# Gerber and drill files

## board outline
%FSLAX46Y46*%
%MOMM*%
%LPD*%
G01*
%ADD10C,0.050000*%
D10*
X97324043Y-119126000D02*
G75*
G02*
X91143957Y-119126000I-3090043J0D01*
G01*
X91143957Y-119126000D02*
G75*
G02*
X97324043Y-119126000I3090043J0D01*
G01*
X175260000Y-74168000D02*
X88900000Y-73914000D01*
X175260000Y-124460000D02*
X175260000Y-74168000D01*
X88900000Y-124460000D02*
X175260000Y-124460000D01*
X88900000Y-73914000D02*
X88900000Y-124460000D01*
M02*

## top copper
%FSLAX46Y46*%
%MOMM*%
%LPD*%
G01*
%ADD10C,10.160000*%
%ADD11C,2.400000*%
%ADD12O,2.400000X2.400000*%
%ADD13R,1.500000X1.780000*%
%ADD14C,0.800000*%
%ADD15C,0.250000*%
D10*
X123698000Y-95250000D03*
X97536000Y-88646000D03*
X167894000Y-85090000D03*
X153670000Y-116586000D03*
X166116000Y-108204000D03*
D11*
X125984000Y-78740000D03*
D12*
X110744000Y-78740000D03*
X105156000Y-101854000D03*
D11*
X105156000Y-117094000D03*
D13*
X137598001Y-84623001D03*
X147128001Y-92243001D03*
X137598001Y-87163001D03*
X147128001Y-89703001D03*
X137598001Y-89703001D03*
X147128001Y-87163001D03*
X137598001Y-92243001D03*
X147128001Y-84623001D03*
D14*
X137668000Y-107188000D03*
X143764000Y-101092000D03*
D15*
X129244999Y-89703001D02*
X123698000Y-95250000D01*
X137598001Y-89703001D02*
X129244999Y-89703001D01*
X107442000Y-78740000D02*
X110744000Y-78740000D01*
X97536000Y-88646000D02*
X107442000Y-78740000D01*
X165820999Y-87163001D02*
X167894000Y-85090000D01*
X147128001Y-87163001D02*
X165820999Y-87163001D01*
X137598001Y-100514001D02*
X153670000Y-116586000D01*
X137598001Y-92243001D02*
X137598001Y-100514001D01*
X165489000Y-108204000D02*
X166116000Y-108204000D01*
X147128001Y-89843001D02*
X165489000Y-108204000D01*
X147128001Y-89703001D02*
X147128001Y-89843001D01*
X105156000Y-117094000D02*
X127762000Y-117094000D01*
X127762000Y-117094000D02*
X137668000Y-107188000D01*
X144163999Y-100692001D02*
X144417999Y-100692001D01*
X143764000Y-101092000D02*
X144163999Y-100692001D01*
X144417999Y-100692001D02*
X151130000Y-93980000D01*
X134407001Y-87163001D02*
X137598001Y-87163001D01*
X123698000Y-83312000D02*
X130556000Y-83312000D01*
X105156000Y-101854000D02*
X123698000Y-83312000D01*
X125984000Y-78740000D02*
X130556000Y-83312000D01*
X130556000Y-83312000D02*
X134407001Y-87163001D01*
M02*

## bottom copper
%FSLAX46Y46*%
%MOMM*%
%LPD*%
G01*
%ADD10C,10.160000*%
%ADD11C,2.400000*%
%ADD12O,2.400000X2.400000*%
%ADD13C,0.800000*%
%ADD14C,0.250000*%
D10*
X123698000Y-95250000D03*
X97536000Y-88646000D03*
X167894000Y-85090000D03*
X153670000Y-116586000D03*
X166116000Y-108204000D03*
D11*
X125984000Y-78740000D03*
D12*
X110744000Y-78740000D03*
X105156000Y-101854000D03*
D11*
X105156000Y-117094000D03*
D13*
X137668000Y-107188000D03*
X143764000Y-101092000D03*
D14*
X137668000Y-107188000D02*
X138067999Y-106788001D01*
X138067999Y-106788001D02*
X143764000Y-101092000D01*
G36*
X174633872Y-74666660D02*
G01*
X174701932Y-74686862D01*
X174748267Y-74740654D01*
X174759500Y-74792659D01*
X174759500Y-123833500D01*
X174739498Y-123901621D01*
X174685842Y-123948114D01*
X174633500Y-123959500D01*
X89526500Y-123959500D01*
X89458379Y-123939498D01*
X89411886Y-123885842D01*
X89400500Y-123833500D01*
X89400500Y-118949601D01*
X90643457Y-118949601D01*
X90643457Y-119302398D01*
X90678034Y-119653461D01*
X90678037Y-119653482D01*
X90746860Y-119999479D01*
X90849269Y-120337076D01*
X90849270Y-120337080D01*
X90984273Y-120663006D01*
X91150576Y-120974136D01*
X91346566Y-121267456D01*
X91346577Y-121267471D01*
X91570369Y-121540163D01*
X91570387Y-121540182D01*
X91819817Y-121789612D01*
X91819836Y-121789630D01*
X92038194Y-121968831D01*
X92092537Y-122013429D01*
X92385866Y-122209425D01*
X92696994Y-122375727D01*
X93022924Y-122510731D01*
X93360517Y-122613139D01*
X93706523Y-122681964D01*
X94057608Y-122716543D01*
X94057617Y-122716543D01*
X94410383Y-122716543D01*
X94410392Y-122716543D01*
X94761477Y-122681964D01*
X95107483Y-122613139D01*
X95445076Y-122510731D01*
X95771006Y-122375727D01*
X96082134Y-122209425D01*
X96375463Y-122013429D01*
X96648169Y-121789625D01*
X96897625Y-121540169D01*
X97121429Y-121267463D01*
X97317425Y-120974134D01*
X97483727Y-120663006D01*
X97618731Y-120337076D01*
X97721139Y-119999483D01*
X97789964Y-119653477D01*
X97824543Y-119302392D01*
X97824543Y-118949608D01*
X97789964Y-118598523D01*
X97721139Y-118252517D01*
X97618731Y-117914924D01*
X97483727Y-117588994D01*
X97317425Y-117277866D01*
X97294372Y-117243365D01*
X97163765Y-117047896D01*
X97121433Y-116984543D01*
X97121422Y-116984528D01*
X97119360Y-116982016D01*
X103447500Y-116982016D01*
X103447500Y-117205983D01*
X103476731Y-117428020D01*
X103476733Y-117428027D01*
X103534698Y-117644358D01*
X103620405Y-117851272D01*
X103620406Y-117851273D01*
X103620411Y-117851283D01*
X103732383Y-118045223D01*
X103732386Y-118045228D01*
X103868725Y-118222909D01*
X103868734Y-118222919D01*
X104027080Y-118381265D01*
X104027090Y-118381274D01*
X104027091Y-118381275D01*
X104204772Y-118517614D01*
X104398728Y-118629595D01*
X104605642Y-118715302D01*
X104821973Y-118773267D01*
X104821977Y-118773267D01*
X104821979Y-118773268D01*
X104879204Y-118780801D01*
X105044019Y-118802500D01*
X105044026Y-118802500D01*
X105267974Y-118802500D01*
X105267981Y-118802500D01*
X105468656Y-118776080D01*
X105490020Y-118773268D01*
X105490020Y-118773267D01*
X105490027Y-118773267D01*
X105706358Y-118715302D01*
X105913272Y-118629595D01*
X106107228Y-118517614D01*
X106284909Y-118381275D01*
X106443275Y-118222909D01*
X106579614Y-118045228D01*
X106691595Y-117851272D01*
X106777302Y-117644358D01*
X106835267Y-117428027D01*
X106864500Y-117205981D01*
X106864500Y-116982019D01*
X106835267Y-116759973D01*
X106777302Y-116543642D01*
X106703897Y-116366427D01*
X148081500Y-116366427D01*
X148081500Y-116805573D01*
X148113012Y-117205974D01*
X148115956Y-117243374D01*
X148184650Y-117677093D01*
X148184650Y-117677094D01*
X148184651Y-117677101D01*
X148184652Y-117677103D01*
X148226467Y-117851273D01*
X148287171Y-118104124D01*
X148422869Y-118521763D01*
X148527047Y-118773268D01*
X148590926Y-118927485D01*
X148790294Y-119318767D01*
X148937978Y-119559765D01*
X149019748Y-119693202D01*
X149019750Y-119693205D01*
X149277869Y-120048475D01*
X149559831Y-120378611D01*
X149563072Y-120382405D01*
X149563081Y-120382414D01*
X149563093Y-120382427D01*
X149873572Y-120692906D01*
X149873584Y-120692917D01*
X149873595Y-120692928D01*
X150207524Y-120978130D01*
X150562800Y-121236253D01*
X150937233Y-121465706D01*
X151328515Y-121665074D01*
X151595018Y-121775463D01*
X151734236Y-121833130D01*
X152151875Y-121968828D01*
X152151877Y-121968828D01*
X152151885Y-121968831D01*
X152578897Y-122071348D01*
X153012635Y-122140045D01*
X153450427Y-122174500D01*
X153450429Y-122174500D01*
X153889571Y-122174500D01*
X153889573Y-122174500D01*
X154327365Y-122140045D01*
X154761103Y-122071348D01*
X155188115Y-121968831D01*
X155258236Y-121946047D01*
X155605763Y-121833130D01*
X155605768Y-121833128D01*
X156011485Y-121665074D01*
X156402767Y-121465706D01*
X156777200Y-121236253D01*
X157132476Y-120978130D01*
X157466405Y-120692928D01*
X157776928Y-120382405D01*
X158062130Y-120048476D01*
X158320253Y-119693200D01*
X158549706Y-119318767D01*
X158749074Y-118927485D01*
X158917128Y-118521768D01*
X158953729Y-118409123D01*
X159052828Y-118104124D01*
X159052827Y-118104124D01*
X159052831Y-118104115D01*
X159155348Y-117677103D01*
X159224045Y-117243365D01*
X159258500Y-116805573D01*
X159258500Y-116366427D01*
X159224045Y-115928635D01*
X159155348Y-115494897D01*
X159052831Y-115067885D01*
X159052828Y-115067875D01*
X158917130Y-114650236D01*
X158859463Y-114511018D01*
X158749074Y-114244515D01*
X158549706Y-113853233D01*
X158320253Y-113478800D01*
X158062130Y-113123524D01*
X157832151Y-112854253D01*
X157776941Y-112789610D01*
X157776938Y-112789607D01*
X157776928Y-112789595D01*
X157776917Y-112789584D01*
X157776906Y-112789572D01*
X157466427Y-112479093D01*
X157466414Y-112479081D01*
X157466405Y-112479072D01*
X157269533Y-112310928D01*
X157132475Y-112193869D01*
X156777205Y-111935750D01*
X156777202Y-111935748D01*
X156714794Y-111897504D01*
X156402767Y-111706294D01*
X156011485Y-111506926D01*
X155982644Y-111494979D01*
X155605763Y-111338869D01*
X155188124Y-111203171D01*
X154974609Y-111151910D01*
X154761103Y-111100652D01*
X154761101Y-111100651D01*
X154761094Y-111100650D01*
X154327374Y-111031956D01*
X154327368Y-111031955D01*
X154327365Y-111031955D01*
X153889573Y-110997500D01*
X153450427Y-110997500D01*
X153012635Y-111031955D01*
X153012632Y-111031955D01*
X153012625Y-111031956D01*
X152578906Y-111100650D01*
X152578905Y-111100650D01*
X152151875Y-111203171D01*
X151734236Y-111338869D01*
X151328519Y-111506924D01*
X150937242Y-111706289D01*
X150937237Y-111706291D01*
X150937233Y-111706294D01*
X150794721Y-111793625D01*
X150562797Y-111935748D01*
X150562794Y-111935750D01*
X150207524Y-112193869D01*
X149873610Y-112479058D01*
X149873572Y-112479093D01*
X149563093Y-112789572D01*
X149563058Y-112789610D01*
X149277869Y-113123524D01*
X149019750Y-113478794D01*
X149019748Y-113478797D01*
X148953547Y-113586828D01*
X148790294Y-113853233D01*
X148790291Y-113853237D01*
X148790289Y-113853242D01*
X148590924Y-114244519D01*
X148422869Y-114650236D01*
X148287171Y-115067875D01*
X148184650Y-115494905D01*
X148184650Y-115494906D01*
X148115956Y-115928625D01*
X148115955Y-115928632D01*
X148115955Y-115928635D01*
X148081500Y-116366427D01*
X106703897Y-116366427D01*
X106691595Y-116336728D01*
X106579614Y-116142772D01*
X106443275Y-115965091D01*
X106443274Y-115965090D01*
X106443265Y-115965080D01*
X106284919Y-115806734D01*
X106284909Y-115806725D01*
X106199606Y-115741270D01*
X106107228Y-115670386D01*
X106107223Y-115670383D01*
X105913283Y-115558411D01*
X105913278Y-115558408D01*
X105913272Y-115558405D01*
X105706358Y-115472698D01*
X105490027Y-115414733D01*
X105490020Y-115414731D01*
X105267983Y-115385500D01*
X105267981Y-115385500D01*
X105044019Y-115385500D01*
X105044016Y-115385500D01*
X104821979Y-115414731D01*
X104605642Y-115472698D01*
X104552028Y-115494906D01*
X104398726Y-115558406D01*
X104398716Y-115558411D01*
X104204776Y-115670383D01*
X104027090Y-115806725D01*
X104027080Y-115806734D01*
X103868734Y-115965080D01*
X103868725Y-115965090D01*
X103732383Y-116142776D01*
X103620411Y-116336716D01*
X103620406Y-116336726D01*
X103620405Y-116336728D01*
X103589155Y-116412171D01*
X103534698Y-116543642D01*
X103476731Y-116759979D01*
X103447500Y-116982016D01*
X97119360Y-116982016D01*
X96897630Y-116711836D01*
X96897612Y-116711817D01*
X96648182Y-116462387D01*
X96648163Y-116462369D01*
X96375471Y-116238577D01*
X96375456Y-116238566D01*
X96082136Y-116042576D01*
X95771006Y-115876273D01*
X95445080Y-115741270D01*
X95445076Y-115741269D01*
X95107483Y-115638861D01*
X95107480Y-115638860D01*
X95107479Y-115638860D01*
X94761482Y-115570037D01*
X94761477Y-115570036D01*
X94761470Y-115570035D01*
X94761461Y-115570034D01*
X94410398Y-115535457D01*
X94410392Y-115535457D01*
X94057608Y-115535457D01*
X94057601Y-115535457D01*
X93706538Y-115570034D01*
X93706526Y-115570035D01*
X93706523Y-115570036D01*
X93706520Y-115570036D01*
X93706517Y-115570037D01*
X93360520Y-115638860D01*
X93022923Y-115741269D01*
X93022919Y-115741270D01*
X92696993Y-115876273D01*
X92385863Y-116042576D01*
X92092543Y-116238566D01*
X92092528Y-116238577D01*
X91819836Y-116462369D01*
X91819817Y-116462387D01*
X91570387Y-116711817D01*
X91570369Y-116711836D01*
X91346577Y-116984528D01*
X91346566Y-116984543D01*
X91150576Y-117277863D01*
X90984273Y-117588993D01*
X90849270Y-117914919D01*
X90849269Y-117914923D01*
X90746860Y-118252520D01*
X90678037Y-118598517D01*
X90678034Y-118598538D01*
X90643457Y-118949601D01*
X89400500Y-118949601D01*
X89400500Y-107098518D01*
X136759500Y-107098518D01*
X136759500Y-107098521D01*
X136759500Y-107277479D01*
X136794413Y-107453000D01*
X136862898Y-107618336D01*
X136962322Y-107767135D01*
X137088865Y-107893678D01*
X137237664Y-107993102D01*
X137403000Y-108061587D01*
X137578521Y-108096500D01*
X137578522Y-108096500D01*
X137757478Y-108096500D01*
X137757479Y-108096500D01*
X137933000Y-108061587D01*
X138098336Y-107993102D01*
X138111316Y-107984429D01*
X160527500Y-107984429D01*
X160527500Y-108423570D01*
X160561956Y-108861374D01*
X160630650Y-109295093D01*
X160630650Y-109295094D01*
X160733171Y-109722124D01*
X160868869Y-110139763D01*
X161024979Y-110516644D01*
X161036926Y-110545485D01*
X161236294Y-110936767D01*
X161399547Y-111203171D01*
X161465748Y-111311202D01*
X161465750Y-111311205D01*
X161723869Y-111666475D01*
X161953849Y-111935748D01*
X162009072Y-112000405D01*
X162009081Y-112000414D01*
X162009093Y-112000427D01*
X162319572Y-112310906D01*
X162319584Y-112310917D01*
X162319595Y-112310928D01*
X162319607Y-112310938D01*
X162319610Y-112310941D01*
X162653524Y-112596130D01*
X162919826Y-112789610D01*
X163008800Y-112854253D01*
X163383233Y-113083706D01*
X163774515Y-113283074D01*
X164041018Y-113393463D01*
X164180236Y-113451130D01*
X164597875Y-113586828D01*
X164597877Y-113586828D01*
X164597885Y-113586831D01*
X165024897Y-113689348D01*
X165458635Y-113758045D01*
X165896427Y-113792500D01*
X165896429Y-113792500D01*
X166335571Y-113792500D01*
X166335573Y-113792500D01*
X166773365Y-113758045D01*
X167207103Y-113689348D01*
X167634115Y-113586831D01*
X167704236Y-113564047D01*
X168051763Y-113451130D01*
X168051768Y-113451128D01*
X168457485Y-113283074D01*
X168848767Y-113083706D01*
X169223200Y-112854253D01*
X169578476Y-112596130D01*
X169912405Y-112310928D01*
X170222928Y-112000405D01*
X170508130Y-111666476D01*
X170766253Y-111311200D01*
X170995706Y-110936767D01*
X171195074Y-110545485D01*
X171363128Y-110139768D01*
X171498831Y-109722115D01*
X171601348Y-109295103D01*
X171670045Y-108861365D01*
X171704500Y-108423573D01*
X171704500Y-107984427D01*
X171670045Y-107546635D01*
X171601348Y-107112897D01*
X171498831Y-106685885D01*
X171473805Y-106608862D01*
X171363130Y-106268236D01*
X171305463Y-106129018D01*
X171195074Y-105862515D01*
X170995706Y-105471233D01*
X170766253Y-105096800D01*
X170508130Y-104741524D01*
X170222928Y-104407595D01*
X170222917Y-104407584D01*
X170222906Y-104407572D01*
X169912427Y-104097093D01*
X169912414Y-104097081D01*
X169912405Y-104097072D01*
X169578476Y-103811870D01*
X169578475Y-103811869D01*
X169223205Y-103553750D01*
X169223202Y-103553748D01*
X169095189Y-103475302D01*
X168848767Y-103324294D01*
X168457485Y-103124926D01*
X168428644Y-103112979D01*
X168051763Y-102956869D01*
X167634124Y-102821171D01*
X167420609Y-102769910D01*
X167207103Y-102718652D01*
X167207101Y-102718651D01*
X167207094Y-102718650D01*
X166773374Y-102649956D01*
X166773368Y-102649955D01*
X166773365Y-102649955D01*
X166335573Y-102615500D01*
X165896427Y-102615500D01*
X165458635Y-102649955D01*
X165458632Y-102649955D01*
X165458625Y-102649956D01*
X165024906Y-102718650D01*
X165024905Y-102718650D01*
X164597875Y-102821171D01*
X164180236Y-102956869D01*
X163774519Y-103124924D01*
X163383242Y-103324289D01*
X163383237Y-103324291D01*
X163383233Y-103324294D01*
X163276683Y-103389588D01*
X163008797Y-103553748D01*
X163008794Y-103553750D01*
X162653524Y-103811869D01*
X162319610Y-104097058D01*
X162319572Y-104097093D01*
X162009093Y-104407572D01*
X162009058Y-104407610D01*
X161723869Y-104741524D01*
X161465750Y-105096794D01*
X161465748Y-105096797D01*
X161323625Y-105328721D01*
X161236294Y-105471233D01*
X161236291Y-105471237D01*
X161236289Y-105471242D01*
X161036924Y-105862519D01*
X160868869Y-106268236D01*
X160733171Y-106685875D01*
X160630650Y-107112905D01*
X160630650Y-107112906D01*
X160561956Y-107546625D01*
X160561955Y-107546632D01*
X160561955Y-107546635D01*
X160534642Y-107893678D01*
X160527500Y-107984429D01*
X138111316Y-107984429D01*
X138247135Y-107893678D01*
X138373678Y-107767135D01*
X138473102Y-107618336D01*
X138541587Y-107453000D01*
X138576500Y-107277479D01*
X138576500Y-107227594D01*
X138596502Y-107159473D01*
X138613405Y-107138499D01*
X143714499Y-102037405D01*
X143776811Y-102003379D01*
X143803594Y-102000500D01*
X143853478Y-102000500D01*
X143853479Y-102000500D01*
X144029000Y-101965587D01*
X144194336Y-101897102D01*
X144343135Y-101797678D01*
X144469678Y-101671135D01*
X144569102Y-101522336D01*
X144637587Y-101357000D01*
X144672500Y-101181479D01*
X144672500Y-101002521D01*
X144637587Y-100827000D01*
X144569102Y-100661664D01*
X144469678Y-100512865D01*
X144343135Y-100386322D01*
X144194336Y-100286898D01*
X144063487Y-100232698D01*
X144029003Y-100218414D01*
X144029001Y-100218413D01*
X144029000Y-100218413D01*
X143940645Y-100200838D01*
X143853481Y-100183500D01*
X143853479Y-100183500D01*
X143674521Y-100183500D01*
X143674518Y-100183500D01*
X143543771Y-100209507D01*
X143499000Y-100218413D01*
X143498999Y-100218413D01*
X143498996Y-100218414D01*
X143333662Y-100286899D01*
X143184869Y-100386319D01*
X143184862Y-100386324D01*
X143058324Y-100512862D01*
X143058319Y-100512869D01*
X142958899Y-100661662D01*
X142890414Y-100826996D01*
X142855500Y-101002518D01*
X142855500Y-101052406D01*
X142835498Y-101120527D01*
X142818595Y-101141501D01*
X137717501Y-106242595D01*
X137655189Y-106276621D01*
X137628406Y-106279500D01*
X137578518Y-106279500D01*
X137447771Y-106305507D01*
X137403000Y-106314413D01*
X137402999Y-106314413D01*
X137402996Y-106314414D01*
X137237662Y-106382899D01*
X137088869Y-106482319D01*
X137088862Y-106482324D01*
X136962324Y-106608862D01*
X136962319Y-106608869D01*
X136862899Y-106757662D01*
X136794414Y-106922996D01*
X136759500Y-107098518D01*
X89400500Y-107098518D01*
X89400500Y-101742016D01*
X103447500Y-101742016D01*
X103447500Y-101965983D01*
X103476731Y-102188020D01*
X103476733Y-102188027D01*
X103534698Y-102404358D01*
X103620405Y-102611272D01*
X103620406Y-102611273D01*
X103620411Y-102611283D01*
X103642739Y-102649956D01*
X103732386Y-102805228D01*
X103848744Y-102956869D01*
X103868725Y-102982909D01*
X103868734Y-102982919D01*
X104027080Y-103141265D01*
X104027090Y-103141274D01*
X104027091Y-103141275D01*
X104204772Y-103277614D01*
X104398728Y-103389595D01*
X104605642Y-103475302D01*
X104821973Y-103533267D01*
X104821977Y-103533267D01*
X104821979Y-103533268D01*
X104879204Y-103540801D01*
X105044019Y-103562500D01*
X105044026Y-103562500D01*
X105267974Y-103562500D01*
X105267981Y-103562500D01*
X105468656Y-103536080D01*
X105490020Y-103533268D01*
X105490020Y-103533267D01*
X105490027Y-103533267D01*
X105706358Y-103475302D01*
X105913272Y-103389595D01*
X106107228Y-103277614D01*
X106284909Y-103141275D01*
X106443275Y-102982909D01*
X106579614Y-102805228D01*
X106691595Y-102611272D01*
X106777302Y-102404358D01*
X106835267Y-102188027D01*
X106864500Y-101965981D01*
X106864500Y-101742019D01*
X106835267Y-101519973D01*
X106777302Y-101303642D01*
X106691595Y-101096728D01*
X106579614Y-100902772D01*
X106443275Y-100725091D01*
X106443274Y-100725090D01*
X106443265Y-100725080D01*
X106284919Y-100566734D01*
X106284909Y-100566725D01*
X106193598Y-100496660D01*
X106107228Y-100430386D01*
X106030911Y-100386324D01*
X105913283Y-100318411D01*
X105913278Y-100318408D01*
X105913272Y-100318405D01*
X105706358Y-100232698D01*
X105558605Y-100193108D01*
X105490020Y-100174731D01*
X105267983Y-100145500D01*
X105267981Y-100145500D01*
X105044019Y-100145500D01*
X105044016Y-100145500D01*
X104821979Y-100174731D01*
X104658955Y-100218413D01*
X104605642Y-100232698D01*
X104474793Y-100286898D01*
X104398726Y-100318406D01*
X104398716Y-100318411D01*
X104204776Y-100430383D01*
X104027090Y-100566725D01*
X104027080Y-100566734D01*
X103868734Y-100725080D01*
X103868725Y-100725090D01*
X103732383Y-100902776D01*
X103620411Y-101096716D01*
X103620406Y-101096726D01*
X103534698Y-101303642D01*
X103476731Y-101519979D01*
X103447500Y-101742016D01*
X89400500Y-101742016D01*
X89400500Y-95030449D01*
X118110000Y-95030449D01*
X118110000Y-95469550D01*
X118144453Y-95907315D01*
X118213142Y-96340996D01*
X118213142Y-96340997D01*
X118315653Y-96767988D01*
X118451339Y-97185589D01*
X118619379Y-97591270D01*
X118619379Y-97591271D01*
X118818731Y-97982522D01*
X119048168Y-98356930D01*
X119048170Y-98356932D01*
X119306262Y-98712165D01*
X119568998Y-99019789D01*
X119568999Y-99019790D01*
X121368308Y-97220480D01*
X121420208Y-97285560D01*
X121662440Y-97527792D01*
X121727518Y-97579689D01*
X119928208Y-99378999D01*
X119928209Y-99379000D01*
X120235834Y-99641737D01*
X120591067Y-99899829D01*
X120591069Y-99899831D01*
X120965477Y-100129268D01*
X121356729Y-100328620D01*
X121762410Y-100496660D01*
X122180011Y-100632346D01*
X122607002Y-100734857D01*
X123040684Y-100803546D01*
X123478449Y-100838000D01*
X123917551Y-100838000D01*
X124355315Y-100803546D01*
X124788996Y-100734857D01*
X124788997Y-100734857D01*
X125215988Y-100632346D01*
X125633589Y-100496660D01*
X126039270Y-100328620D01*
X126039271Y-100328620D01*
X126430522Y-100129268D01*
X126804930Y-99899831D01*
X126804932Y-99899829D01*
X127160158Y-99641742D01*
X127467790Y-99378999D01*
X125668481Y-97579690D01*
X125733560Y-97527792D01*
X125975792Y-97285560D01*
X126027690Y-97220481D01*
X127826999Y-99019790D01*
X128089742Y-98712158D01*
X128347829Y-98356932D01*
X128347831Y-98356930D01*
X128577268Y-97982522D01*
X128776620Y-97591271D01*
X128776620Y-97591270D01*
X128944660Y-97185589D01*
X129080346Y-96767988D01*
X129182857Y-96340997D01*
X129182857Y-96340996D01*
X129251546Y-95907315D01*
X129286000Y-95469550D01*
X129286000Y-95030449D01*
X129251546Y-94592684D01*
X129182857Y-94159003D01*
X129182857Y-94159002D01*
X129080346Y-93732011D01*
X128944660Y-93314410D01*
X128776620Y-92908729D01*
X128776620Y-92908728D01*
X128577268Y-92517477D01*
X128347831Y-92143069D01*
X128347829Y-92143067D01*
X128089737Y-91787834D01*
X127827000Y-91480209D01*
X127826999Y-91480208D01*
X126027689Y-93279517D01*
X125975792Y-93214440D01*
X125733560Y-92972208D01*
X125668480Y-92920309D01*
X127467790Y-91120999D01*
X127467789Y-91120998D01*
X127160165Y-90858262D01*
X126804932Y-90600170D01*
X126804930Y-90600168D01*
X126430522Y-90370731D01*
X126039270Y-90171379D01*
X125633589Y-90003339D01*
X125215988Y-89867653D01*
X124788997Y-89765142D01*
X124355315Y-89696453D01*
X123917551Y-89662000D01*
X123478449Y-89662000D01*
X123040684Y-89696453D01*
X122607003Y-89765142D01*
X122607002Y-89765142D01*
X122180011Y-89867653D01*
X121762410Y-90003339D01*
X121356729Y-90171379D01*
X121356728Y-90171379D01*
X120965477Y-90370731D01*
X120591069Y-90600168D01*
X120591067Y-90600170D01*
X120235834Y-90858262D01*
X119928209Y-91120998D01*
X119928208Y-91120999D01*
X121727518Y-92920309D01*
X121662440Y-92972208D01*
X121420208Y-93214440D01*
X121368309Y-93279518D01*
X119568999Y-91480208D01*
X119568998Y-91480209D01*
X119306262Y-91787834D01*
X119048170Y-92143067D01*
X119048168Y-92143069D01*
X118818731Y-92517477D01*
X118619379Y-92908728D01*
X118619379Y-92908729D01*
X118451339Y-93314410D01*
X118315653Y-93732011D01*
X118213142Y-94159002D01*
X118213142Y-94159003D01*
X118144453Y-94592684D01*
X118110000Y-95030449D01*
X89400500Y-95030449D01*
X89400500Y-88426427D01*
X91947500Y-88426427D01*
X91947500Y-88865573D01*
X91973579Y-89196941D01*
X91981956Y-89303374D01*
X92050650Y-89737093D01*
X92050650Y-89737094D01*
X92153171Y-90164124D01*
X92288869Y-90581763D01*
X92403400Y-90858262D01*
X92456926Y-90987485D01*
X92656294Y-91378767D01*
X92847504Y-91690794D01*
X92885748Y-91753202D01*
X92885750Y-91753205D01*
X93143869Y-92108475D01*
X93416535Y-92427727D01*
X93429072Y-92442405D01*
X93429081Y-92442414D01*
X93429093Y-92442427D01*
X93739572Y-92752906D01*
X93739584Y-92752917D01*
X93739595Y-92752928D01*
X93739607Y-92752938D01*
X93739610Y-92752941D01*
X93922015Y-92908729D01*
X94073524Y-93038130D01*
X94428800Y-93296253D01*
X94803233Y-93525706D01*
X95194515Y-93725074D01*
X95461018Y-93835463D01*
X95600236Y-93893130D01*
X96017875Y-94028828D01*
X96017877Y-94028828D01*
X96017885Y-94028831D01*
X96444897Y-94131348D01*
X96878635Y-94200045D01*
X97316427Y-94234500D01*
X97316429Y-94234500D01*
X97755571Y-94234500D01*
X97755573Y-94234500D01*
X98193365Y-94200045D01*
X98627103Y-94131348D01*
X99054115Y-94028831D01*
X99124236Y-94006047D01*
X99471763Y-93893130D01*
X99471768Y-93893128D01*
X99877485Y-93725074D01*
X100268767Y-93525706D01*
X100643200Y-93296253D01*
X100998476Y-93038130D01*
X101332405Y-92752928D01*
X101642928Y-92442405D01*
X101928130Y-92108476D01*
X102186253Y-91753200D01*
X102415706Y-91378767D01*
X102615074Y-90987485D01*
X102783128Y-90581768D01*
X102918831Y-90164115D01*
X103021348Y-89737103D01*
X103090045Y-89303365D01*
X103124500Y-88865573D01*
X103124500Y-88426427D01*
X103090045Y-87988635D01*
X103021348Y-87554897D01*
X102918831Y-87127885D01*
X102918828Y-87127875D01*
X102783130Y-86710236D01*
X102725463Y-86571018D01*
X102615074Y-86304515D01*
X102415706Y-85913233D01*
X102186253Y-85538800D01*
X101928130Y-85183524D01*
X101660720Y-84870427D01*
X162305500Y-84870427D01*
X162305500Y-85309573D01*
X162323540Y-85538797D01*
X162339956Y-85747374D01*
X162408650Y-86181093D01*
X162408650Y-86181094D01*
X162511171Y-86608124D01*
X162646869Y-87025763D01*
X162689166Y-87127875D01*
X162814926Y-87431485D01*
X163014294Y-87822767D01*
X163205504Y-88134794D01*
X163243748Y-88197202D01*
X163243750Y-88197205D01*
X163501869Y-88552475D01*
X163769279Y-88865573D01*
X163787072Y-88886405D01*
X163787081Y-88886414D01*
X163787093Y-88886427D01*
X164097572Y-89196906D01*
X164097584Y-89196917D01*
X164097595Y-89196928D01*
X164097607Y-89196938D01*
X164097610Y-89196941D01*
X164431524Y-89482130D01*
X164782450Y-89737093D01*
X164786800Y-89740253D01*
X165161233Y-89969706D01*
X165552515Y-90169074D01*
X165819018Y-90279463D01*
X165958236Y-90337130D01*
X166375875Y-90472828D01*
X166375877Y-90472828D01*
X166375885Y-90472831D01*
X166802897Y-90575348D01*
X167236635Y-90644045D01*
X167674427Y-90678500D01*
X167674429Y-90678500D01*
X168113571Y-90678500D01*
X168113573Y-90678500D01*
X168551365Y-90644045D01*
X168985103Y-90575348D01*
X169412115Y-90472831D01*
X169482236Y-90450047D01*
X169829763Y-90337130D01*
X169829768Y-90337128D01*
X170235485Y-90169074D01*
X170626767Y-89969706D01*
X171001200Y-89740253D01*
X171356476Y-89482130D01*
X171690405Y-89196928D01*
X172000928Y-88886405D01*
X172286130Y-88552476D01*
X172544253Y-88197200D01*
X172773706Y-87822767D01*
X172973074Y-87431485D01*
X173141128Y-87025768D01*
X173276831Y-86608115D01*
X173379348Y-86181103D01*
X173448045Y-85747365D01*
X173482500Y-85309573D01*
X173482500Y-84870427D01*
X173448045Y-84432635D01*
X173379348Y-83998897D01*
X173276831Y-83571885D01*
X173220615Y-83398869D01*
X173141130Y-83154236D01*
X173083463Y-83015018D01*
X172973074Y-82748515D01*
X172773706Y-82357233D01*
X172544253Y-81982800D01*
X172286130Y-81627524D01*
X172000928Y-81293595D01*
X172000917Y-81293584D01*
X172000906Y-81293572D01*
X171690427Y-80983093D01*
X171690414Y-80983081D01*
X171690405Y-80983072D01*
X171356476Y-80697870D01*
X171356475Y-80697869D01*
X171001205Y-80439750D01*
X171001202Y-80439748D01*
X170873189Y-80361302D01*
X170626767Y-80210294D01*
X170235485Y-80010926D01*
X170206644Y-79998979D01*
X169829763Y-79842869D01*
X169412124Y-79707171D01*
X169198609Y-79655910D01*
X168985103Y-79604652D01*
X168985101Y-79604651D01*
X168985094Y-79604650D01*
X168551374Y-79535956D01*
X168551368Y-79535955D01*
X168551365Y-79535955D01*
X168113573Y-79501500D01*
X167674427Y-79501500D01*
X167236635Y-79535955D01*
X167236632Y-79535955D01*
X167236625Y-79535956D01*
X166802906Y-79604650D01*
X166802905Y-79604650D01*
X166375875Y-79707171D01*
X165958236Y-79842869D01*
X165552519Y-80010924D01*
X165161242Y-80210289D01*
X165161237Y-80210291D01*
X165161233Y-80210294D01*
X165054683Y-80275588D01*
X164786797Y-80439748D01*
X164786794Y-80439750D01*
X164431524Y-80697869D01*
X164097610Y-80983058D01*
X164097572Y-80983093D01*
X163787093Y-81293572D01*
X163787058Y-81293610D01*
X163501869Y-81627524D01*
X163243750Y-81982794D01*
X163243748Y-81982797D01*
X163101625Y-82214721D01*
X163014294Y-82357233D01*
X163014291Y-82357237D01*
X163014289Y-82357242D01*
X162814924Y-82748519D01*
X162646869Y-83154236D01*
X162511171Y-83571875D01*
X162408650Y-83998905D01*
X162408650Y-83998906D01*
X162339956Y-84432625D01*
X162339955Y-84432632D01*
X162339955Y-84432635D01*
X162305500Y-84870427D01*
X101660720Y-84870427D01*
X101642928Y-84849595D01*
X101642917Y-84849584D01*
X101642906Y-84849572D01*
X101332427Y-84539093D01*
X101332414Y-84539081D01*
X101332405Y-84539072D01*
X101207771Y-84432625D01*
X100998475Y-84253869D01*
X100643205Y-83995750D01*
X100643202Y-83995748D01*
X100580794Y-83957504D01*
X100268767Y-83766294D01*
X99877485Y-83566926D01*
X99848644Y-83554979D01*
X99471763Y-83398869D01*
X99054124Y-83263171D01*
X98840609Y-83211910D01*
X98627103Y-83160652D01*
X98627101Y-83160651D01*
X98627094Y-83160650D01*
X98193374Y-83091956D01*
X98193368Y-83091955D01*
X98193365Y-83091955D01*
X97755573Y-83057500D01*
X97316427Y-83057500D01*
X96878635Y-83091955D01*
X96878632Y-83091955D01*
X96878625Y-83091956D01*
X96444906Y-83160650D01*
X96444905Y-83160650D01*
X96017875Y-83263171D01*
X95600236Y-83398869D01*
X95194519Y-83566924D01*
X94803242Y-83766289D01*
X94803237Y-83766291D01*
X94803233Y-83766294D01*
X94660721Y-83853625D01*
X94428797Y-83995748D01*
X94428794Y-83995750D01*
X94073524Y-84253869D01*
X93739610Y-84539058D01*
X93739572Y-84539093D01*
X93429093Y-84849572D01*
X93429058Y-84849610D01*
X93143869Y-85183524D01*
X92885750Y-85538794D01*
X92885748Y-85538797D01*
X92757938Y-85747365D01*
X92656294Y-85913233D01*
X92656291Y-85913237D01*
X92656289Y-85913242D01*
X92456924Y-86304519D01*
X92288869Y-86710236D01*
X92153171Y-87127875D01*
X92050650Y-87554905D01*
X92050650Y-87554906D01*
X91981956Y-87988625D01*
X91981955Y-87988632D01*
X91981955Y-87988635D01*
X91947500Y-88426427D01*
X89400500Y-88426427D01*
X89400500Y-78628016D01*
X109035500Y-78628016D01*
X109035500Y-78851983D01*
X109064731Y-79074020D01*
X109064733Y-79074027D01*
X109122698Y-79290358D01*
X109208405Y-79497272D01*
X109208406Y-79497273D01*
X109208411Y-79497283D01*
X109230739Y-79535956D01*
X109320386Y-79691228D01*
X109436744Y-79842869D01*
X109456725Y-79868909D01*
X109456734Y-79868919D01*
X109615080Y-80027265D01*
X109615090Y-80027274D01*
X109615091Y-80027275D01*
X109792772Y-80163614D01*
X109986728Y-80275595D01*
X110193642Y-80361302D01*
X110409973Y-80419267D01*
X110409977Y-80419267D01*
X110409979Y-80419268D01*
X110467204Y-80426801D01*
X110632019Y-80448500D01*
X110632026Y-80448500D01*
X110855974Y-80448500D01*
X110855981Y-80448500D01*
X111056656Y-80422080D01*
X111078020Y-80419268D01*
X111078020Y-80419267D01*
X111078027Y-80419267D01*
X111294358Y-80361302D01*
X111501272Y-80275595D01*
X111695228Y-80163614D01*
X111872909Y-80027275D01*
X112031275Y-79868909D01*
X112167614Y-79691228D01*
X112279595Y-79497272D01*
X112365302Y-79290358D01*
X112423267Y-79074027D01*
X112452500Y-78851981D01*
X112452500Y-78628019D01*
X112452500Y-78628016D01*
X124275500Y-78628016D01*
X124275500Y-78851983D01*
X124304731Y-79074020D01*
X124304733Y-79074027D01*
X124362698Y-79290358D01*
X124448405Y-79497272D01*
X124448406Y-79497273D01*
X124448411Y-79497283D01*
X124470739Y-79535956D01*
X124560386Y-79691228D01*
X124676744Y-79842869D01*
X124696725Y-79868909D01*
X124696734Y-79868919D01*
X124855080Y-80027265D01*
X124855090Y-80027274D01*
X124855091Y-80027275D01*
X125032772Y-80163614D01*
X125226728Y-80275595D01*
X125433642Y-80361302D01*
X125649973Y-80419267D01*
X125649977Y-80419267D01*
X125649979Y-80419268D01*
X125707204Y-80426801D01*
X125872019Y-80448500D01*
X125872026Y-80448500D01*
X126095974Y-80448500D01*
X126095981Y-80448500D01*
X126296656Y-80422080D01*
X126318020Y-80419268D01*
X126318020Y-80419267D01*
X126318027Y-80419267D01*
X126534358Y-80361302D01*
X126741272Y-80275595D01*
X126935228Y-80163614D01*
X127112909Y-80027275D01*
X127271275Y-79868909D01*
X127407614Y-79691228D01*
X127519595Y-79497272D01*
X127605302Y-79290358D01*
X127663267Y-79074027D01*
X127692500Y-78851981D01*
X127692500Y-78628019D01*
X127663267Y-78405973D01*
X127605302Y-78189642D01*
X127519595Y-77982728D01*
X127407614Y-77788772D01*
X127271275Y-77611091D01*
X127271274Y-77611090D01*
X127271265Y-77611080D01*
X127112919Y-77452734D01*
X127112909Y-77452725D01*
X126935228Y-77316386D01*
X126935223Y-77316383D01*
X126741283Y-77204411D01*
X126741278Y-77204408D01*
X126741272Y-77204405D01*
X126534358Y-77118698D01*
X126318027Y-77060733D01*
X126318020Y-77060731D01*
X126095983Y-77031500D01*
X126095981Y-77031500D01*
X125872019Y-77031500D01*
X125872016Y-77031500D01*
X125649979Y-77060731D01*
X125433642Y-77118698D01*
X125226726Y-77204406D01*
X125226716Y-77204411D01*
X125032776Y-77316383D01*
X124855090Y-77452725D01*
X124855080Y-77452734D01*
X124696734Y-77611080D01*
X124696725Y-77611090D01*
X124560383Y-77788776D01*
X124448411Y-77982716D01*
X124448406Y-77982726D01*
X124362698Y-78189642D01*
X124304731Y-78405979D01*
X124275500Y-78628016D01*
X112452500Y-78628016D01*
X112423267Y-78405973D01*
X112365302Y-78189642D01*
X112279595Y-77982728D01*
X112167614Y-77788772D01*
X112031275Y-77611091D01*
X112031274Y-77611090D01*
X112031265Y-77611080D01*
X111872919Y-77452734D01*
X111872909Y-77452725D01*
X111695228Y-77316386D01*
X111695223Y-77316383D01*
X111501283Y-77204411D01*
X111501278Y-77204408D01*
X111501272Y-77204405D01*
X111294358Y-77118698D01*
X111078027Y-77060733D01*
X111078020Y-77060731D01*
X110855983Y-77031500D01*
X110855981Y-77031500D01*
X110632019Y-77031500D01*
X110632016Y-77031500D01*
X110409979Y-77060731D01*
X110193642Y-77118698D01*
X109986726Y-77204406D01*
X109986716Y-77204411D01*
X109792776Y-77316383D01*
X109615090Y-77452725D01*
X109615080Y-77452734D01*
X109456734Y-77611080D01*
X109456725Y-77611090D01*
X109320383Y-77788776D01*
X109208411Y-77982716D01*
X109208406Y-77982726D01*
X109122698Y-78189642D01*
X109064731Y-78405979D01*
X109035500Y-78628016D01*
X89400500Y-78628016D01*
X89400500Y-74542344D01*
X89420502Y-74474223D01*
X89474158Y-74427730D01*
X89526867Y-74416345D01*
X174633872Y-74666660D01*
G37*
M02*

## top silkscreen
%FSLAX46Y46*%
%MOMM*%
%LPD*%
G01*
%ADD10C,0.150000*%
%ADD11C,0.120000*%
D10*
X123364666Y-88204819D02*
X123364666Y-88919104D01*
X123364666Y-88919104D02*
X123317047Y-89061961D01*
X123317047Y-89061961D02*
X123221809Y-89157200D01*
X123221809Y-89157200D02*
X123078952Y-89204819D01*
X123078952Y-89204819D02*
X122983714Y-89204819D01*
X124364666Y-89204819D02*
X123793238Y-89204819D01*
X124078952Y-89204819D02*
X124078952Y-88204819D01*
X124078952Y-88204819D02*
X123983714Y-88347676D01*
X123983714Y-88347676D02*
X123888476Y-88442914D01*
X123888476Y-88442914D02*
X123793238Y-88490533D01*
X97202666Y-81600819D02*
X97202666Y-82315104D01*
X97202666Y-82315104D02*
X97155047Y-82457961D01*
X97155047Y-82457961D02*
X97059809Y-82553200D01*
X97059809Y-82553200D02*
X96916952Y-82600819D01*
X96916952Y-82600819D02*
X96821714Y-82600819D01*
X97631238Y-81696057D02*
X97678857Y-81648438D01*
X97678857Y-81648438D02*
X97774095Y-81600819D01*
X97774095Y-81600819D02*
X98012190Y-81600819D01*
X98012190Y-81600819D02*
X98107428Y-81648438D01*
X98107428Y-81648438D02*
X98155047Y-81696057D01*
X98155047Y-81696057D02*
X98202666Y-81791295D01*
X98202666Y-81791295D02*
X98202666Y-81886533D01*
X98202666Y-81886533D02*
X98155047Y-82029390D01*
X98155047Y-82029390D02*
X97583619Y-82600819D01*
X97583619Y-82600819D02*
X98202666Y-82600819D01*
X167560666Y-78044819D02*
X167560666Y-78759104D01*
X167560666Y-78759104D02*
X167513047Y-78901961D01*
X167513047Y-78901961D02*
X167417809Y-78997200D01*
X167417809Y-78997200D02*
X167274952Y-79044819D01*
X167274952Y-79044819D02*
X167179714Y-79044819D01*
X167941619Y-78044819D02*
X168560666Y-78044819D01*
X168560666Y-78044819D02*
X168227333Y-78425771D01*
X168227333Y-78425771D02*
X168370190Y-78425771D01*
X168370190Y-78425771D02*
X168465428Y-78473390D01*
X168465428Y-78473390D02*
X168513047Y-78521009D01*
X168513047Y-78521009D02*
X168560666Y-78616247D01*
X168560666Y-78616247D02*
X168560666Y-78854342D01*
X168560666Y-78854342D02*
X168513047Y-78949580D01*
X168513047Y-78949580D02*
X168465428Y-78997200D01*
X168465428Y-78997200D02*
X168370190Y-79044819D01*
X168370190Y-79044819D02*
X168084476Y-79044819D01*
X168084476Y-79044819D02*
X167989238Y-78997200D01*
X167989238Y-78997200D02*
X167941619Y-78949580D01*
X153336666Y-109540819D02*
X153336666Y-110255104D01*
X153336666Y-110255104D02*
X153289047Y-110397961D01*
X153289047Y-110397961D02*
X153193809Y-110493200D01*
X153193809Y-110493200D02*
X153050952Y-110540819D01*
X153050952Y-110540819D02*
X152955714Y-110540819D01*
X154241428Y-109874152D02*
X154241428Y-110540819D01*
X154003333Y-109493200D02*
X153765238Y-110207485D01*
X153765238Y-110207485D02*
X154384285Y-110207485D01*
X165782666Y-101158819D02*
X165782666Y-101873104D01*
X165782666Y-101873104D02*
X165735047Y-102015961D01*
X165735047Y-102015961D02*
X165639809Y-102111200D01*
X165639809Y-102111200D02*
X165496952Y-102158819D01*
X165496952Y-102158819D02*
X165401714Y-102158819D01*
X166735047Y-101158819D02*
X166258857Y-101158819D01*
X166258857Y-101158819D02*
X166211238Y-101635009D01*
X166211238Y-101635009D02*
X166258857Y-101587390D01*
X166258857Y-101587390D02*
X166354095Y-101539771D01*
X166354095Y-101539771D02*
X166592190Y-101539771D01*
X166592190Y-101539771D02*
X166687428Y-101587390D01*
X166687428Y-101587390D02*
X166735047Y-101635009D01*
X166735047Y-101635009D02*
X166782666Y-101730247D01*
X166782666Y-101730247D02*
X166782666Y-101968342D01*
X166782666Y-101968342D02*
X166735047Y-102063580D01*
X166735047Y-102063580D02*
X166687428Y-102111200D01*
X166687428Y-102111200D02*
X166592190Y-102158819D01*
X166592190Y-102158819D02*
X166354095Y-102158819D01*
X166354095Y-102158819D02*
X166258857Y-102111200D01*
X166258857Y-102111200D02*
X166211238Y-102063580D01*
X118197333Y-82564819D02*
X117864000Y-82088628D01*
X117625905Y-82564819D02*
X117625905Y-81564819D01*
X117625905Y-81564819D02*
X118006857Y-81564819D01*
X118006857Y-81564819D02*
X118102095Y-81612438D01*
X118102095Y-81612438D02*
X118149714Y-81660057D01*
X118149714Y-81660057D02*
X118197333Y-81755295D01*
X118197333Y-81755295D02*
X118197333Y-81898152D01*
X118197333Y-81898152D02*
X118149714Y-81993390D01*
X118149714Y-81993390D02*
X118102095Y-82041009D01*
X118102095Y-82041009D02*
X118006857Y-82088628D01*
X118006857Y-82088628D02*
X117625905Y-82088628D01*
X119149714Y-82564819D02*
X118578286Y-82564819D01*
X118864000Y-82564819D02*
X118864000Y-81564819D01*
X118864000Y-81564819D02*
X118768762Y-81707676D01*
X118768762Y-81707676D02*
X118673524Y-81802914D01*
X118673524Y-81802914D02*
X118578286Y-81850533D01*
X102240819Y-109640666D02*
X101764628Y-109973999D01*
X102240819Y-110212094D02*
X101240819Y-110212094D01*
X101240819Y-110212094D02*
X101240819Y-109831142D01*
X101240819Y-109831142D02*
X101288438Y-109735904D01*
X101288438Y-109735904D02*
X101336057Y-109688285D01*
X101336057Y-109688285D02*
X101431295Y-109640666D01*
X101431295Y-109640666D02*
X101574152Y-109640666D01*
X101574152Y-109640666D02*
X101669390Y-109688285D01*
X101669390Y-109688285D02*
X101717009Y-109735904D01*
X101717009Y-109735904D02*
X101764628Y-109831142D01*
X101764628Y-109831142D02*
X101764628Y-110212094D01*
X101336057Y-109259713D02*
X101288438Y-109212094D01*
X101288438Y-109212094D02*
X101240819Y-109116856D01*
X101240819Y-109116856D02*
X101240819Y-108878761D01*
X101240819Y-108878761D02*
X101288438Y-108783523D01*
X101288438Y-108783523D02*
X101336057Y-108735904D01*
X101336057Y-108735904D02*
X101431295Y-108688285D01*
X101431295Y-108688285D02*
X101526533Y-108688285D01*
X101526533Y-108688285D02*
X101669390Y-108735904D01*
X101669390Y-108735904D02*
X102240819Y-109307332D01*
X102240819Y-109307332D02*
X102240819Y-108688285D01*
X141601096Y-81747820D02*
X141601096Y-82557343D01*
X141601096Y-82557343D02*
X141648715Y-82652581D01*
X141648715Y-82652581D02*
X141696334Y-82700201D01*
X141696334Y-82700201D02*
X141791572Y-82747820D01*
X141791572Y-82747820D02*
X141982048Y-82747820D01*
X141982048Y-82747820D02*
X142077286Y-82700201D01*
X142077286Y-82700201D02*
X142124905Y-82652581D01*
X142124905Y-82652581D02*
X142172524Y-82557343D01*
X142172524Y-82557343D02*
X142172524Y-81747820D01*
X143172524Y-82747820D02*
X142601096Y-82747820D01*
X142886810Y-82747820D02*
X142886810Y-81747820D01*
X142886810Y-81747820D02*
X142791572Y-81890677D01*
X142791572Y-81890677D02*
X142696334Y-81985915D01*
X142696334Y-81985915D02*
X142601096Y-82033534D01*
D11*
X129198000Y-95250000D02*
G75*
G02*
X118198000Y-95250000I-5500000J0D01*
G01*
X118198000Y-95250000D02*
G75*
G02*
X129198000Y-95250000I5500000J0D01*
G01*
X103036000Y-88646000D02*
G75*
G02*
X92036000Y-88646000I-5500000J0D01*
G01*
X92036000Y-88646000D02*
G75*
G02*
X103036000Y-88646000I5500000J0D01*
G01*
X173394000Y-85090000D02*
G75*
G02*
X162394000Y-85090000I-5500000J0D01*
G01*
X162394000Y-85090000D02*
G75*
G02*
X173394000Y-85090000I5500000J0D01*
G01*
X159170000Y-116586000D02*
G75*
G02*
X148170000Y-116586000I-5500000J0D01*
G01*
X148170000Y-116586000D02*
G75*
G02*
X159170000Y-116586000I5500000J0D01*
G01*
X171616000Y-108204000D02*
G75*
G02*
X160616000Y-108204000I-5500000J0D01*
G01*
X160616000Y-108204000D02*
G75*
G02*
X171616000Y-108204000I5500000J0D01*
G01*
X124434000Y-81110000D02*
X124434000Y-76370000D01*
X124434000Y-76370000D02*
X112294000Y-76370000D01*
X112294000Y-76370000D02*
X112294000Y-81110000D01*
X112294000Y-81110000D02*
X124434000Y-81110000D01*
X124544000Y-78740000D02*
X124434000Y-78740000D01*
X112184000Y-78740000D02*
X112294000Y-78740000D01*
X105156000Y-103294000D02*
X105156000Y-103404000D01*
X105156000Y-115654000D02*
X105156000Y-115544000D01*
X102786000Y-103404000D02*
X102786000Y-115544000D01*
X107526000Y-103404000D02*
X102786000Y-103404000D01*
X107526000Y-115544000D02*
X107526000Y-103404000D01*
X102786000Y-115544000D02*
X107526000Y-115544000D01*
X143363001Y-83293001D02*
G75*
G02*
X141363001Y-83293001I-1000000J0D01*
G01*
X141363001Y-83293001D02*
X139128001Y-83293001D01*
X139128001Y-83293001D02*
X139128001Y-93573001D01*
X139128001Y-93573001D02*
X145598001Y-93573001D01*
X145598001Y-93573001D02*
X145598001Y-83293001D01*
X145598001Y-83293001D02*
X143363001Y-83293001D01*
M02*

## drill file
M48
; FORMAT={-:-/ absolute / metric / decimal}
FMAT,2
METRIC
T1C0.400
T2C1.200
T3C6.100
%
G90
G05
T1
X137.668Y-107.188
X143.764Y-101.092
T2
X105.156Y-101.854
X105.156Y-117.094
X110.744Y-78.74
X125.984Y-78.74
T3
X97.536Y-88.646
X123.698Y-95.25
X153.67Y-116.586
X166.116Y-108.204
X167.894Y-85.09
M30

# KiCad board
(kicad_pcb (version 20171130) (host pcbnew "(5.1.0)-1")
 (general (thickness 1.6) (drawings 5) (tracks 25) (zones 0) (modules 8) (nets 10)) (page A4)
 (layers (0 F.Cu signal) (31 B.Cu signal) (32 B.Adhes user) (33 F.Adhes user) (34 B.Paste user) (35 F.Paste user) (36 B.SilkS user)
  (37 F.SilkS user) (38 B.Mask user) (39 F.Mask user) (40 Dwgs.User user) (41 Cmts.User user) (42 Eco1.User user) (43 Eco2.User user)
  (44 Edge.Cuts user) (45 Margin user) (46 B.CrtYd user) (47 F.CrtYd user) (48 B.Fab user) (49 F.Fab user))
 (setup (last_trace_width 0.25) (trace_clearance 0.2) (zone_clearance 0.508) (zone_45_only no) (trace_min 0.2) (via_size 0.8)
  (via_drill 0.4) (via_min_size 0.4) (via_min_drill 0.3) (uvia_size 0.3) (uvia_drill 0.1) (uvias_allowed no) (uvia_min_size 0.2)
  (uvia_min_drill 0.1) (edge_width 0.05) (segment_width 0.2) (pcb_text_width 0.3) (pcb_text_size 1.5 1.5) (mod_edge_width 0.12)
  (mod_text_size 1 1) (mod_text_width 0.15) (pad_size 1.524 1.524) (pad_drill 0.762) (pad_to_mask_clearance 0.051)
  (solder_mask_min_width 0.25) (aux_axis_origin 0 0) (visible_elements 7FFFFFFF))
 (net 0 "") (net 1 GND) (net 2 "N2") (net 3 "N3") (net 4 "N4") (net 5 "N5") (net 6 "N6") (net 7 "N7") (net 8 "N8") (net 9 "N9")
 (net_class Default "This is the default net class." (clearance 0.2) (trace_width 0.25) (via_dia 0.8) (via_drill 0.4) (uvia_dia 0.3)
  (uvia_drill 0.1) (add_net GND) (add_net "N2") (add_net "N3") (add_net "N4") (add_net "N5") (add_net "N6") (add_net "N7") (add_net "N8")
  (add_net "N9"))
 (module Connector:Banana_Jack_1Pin (layer F.Cu) (at 123.698 95.25)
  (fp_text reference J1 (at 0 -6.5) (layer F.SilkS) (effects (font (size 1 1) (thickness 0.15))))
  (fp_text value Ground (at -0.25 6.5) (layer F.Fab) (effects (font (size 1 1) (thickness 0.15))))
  (fp_circle (center 0 0) (end 5.5 0) (layer F.SilkS) (width 0.12))
  (pad 1 thru_hole circle (at 0 0) (size 10.16 10.16) (drill 6.1) (layers *.Cu *.Mask) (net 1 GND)))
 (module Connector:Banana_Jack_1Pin (layer F.Cu) (at 97.536 88.646)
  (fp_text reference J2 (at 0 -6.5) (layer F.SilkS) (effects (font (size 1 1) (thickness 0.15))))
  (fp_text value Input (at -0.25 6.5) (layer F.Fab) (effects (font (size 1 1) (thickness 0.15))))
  (fp_circle (center 0 0) (end 5.5 0) (layer F.SilkS) (width 0.12))
  (pad 1 thru_hole circle (at 0 0) (size 10.16 10.16) (drill 6.1) (layers *.Cu *.Mask) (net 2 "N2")))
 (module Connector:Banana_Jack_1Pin (layer F.Cu) (at 167.894 85.09)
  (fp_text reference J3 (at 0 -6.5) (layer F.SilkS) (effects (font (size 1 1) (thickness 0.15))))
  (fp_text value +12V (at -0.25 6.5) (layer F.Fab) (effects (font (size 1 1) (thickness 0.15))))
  (fp_circle (center 0 0) (end 5.5 0) (layer F.SilkS) (width 0.12))
  (pad 1 thru_hole circle (at 0 0) (size 10.16 10.16) (drill 6.1) (layers *.Cu *.Mask) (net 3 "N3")))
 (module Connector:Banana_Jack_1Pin (layer F.Cu) (at 153.67 116.586)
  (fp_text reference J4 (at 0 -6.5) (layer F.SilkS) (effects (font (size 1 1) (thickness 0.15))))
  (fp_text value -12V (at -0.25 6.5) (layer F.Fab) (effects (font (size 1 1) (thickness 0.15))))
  (fp_circle (center 0 0) (end 5.5 0) (layer F.SilkS) (width 0.12))
  (pad 1 thru_hole circle (at 0 0) (size 10.16 10.16) (drill 6.1) (layers *.Cu *.Mask) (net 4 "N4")))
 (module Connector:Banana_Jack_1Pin (layer F.Cu) (at 166.116 108.204)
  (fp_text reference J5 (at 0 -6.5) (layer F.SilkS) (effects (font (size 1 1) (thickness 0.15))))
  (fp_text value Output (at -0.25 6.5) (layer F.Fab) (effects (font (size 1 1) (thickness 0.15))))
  (fp_circle (center 0 0) (end 5.5 0) (layer F.SilkS) (width 0.12))
  (pad 1 thru_hole circle (at 0 0) (size 10.16 10.16) (drill 6.1) (layers *.Cu *.Mask) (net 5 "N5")))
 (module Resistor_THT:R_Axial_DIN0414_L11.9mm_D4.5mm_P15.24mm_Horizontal (layer F.Cu) (at 125.984 78.74 180)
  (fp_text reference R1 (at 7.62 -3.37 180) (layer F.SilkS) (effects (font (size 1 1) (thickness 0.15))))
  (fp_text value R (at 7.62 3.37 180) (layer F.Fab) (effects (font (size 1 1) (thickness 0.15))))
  (fp_line (start 1.55 -2.37) (end 1.55 2.37) (layer F.SilkS) (width 0.12))
  (fp_line (start 1.55 2.37) (end 13.69 2.37) (layer F.SilkS) (width 0.12))
  (fp_line (start 13.69 2.37) (end 13.69 -2.37) (layer F.SilkS) (width 0.12))
  (fp_line (start 13.69 -2.37) (end 1.55 -2.37) (layer F.SilkS) (width 0.12))
  (fp_line (start 1.44 0) (end 1.55 0) (layer F.SilkS) (width 0.12))
  (fp_line (start 13.8 0) (end 13.69 0) (layer F.SilkS) (width 0.12))
  (pad 1 thru_hole circle (at 0 0 180) (size 2.4 2.4) (drill 1.2) (layers *.Cu *.Mask) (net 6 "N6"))
  (pad 2 thru_hole oval (at 15.24 0 180) (size 2.4 2.4) (drill 1.2) (layers *.Cu *.Mask) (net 2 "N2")))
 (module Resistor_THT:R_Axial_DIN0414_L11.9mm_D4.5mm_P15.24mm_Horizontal (layer F.Cu) (at 105.156 117.094 90)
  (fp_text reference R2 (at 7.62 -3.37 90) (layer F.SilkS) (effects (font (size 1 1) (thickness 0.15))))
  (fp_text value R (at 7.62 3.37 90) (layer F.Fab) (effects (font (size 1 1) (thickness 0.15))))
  (fp_line (start 13.8 0) (end 13.69 0) (layer F.SilkS) (width 0.12))
  (fp_line (start 1.44 0) (end 1.55 0) (layer F.SilkS) (width 0.12))
  (fp_line (start 13.69 -2.37) (end 1.55 -2.37) (layer F.SilkS) (width 0.12))
  (fp_line (start 13.69 2.37) (end 13.69 -2.37) (layer F.SilkS) (width 0.12))
  (fp_line (start 1.55 2.37) (end 13.69 2.37) (layer F.SilkS) (width 0.12))
  (fp_line (start 1.55 -2.37) (end 1.55 2.37) (layer F.SilkS) (width 0.12))
  (pad 2 thru_hole oval (at 15.24 0 90) (size 2.4 2.4) (drill 1.2) (layers *.Cu *.Mask) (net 6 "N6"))
  (pad 1 thru_hole circle (at 0 0 90) (size 2.4 2.4) (drill 1.2) (layers *.Cu *.Mask) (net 5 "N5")))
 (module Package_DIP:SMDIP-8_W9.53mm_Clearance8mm (layer F.Cu) (at 142.363001 88.433001)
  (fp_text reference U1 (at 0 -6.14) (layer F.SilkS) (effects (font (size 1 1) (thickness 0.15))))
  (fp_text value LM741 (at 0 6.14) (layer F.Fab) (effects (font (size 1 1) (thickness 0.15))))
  (fp_arc (start 0 -5.14) (end -1 -5.14) (angle -180) (layer F.SilkS) (width 0.12))
  (fp_line (start -1 -5.14) (end -3.235 -5.14) (layer F.SilkS) (width 0.12))
  (fp_line (start -3.235 -5.14) (end -3.235 5.14) (layer F.SilkS) (width 0.12))
  (fp_line (start -3.235 5.14) (end 3.235 5.14) (layer F.SilkS) (width 0.12))
  (fp_line (start 3.235 5.14) (end 3.235 -5.14) (layer F.SilkS) (width 0.12))
  (fp_line (start 3.235 -5.14) (end 1 -5.14) (layer F.SilkS) (width 0.12))
  (pad 1 smd rect (at -4.765 -3.81) (size 1.5 1.78) (layers F.Cu F.Paste F.Mask) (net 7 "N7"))
  (pad 5 smd rect (at 4.765 3.81) (size 1.5 1.78) (layers F.Cu F.Paste F.Mask) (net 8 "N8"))
  (pad 2 smd rect (at -4.765 -1.27) (size 1.5 1.78) (layers F.Cu F.Paste F.Mask) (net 6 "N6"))
  (pad 6 smd rect (at 4.765 1.27) (size 1.5 1.78) (layers F.Cu F.Paste F.Mask) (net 5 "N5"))
  (pad 3 smd rect (at -4.765 1.27) (size 1.5 1.78) (layers F.Cu F.Paste F.Mask) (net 1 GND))
  (pad 7 smd rect (at 4.765 -1.27) (size 1.5 1.78) (layers F.Cu F.Paste F.Mask) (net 3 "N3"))
  (pad 4 smd rect (at -4.765 3.81) (size 1.5 1.78) (layers F.Cu F.Paste F.Mask) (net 4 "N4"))
  (pad 8 smd rect (at 4.765 -3.81) (size 1.5 1.78) (layers F.Cu F.Paste F.Mask) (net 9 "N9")))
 (gr_circle (center 94.234 119.126) (end 97.282 119.634) (layer Edge.Cuts) (width 0.05))
 (gr_line (start 175.26 74.168) (end 88.9 73.914) (layer Edge.Cuts) (width 0.05))
 (gr_line (start 175.26 124.46) (end 175.26 74.168) (layer Edge.Cuts) (width 0.05))
 (gr_line (start 88.9 124.46) (end 175.26 124.46) (layer Edge.Cuts) (width 0.05))
 (gr_line (start 88.9 73.914) (end 88.9 124.46) (layer Edge.Cuts) (width 0.05))
 (segment (start 129.244999 89.703001) (end 123.698 95.25) (width 0.25) (layer F.Cu) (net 1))
 (segment (start 137.598001 89.703001) (end 129.244999 89.703001) (width 0.25) (layer F.Cu) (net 1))
 (segment (start 107.442 78.74) (end 110.744 78.74) (width 0.25) (layer F.Cu) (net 2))
 (segment (start 97.536 88.646) (end 107.442 78.74) (width 0.25) (layer F.Cu) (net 2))
 (segment (start 165.820999 87.163001) (end 167.894 85.09) (width 0.25) (layer F.Cu) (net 3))
 (segment (start 147.128001 87.163001) (end 165.820999 87.163001) (width 0.25) (layer F.Cu) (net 3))
 (segment (start 137.598001 100.514001) (end 153.67 116.586) (width 0.25) (layer F.Cu) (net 4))
 (segment (start 137.598001 92.243001) (end 137.598001 100.514001) (width 0.25) (layer F.Cu) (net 4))
 (segment (start 165.489 108.204) (end 166.116 108.204) (width 0.25) (layer F.Cu) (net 5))
 (segment (start 147.128001 89.843001) (end 165.489 108.204) (width 0.25) (layer F.Cu) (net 5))
 (segment (start 147.128001 89.703001) (end 147.128001 89.843001) (width 0.25) (layer F.Cu) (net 5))
 (segment (start 105.156 117.094) (end 127.762 117.094) (width 0.25) (layer F.Cu) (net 5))
 (segment (start 127.762 117.094) (end 137.668 107.188) (width 0.25) (layer F.Cu) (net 5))
 (via (at 137.668 107.188) (size 0.8) (drill 0.4) (layers F.Cu B.Cu) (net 5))
 (segment (start 137.668 107.188) (end 138.067999 106.788001) (width 0.25) (layer B.Cu) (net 5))
 (segment (start 138.067999 106.788001) (end 143.764 101.092) (width 0.25) (layer B.Cu) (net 5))
 (via (at 143.764 101.092) (size 0.8) (drill 0.4) (layers F.Cu B.Cu) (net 5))
 (segment (start 144.163999 100.692001) (end 144.417999 100.692001) (width 0.25) (layer F.Cu) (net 5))
 (segment (start 143.764 101.092) (end 144.163999 100.692001) (width 0.25) (layer F.Cu) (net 5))
 (segment (start 144.417999 100.692001) (end 151.13 93.98) (width 0.25) (layer F.Cu) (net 5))
 (segment (start 134.407001 87.163001) (end 137.598001 87.163001) (width 0.25) (layer F.Cu) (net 6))
 (segment (start 123.698 83.312) (end 130.556 83.312) (width 0.25) (layer F.Cu) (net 6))
 (segment (start 105.156 101.854) (end 123.698 83.312) (width 0.25) (layer F.Cu) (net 6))
 (segment (start 125.984 78.74) (end 130.556 83.312) (width 0.25) (layer F.Cu) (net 6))
 (segment (start 130.556 83.312) (end 134.407001 87.163001) (width 0.25) (layer F.Cu) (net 6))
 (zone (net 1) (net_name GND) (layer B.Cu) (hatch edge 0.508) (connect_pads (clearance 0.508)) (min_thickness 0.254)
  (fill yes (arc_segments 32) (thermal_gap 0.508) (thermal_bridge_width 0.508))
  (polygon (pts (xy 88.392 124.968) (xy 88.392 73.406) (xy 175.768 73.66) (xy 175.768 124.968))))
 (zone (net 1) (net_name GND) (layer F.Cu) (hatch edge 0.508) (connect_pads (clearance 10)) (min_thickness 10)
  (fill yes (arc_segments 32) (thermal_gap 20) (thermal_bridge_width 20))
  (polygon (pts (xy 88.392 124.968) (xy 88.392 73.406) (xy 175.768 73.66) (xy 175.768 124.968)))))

